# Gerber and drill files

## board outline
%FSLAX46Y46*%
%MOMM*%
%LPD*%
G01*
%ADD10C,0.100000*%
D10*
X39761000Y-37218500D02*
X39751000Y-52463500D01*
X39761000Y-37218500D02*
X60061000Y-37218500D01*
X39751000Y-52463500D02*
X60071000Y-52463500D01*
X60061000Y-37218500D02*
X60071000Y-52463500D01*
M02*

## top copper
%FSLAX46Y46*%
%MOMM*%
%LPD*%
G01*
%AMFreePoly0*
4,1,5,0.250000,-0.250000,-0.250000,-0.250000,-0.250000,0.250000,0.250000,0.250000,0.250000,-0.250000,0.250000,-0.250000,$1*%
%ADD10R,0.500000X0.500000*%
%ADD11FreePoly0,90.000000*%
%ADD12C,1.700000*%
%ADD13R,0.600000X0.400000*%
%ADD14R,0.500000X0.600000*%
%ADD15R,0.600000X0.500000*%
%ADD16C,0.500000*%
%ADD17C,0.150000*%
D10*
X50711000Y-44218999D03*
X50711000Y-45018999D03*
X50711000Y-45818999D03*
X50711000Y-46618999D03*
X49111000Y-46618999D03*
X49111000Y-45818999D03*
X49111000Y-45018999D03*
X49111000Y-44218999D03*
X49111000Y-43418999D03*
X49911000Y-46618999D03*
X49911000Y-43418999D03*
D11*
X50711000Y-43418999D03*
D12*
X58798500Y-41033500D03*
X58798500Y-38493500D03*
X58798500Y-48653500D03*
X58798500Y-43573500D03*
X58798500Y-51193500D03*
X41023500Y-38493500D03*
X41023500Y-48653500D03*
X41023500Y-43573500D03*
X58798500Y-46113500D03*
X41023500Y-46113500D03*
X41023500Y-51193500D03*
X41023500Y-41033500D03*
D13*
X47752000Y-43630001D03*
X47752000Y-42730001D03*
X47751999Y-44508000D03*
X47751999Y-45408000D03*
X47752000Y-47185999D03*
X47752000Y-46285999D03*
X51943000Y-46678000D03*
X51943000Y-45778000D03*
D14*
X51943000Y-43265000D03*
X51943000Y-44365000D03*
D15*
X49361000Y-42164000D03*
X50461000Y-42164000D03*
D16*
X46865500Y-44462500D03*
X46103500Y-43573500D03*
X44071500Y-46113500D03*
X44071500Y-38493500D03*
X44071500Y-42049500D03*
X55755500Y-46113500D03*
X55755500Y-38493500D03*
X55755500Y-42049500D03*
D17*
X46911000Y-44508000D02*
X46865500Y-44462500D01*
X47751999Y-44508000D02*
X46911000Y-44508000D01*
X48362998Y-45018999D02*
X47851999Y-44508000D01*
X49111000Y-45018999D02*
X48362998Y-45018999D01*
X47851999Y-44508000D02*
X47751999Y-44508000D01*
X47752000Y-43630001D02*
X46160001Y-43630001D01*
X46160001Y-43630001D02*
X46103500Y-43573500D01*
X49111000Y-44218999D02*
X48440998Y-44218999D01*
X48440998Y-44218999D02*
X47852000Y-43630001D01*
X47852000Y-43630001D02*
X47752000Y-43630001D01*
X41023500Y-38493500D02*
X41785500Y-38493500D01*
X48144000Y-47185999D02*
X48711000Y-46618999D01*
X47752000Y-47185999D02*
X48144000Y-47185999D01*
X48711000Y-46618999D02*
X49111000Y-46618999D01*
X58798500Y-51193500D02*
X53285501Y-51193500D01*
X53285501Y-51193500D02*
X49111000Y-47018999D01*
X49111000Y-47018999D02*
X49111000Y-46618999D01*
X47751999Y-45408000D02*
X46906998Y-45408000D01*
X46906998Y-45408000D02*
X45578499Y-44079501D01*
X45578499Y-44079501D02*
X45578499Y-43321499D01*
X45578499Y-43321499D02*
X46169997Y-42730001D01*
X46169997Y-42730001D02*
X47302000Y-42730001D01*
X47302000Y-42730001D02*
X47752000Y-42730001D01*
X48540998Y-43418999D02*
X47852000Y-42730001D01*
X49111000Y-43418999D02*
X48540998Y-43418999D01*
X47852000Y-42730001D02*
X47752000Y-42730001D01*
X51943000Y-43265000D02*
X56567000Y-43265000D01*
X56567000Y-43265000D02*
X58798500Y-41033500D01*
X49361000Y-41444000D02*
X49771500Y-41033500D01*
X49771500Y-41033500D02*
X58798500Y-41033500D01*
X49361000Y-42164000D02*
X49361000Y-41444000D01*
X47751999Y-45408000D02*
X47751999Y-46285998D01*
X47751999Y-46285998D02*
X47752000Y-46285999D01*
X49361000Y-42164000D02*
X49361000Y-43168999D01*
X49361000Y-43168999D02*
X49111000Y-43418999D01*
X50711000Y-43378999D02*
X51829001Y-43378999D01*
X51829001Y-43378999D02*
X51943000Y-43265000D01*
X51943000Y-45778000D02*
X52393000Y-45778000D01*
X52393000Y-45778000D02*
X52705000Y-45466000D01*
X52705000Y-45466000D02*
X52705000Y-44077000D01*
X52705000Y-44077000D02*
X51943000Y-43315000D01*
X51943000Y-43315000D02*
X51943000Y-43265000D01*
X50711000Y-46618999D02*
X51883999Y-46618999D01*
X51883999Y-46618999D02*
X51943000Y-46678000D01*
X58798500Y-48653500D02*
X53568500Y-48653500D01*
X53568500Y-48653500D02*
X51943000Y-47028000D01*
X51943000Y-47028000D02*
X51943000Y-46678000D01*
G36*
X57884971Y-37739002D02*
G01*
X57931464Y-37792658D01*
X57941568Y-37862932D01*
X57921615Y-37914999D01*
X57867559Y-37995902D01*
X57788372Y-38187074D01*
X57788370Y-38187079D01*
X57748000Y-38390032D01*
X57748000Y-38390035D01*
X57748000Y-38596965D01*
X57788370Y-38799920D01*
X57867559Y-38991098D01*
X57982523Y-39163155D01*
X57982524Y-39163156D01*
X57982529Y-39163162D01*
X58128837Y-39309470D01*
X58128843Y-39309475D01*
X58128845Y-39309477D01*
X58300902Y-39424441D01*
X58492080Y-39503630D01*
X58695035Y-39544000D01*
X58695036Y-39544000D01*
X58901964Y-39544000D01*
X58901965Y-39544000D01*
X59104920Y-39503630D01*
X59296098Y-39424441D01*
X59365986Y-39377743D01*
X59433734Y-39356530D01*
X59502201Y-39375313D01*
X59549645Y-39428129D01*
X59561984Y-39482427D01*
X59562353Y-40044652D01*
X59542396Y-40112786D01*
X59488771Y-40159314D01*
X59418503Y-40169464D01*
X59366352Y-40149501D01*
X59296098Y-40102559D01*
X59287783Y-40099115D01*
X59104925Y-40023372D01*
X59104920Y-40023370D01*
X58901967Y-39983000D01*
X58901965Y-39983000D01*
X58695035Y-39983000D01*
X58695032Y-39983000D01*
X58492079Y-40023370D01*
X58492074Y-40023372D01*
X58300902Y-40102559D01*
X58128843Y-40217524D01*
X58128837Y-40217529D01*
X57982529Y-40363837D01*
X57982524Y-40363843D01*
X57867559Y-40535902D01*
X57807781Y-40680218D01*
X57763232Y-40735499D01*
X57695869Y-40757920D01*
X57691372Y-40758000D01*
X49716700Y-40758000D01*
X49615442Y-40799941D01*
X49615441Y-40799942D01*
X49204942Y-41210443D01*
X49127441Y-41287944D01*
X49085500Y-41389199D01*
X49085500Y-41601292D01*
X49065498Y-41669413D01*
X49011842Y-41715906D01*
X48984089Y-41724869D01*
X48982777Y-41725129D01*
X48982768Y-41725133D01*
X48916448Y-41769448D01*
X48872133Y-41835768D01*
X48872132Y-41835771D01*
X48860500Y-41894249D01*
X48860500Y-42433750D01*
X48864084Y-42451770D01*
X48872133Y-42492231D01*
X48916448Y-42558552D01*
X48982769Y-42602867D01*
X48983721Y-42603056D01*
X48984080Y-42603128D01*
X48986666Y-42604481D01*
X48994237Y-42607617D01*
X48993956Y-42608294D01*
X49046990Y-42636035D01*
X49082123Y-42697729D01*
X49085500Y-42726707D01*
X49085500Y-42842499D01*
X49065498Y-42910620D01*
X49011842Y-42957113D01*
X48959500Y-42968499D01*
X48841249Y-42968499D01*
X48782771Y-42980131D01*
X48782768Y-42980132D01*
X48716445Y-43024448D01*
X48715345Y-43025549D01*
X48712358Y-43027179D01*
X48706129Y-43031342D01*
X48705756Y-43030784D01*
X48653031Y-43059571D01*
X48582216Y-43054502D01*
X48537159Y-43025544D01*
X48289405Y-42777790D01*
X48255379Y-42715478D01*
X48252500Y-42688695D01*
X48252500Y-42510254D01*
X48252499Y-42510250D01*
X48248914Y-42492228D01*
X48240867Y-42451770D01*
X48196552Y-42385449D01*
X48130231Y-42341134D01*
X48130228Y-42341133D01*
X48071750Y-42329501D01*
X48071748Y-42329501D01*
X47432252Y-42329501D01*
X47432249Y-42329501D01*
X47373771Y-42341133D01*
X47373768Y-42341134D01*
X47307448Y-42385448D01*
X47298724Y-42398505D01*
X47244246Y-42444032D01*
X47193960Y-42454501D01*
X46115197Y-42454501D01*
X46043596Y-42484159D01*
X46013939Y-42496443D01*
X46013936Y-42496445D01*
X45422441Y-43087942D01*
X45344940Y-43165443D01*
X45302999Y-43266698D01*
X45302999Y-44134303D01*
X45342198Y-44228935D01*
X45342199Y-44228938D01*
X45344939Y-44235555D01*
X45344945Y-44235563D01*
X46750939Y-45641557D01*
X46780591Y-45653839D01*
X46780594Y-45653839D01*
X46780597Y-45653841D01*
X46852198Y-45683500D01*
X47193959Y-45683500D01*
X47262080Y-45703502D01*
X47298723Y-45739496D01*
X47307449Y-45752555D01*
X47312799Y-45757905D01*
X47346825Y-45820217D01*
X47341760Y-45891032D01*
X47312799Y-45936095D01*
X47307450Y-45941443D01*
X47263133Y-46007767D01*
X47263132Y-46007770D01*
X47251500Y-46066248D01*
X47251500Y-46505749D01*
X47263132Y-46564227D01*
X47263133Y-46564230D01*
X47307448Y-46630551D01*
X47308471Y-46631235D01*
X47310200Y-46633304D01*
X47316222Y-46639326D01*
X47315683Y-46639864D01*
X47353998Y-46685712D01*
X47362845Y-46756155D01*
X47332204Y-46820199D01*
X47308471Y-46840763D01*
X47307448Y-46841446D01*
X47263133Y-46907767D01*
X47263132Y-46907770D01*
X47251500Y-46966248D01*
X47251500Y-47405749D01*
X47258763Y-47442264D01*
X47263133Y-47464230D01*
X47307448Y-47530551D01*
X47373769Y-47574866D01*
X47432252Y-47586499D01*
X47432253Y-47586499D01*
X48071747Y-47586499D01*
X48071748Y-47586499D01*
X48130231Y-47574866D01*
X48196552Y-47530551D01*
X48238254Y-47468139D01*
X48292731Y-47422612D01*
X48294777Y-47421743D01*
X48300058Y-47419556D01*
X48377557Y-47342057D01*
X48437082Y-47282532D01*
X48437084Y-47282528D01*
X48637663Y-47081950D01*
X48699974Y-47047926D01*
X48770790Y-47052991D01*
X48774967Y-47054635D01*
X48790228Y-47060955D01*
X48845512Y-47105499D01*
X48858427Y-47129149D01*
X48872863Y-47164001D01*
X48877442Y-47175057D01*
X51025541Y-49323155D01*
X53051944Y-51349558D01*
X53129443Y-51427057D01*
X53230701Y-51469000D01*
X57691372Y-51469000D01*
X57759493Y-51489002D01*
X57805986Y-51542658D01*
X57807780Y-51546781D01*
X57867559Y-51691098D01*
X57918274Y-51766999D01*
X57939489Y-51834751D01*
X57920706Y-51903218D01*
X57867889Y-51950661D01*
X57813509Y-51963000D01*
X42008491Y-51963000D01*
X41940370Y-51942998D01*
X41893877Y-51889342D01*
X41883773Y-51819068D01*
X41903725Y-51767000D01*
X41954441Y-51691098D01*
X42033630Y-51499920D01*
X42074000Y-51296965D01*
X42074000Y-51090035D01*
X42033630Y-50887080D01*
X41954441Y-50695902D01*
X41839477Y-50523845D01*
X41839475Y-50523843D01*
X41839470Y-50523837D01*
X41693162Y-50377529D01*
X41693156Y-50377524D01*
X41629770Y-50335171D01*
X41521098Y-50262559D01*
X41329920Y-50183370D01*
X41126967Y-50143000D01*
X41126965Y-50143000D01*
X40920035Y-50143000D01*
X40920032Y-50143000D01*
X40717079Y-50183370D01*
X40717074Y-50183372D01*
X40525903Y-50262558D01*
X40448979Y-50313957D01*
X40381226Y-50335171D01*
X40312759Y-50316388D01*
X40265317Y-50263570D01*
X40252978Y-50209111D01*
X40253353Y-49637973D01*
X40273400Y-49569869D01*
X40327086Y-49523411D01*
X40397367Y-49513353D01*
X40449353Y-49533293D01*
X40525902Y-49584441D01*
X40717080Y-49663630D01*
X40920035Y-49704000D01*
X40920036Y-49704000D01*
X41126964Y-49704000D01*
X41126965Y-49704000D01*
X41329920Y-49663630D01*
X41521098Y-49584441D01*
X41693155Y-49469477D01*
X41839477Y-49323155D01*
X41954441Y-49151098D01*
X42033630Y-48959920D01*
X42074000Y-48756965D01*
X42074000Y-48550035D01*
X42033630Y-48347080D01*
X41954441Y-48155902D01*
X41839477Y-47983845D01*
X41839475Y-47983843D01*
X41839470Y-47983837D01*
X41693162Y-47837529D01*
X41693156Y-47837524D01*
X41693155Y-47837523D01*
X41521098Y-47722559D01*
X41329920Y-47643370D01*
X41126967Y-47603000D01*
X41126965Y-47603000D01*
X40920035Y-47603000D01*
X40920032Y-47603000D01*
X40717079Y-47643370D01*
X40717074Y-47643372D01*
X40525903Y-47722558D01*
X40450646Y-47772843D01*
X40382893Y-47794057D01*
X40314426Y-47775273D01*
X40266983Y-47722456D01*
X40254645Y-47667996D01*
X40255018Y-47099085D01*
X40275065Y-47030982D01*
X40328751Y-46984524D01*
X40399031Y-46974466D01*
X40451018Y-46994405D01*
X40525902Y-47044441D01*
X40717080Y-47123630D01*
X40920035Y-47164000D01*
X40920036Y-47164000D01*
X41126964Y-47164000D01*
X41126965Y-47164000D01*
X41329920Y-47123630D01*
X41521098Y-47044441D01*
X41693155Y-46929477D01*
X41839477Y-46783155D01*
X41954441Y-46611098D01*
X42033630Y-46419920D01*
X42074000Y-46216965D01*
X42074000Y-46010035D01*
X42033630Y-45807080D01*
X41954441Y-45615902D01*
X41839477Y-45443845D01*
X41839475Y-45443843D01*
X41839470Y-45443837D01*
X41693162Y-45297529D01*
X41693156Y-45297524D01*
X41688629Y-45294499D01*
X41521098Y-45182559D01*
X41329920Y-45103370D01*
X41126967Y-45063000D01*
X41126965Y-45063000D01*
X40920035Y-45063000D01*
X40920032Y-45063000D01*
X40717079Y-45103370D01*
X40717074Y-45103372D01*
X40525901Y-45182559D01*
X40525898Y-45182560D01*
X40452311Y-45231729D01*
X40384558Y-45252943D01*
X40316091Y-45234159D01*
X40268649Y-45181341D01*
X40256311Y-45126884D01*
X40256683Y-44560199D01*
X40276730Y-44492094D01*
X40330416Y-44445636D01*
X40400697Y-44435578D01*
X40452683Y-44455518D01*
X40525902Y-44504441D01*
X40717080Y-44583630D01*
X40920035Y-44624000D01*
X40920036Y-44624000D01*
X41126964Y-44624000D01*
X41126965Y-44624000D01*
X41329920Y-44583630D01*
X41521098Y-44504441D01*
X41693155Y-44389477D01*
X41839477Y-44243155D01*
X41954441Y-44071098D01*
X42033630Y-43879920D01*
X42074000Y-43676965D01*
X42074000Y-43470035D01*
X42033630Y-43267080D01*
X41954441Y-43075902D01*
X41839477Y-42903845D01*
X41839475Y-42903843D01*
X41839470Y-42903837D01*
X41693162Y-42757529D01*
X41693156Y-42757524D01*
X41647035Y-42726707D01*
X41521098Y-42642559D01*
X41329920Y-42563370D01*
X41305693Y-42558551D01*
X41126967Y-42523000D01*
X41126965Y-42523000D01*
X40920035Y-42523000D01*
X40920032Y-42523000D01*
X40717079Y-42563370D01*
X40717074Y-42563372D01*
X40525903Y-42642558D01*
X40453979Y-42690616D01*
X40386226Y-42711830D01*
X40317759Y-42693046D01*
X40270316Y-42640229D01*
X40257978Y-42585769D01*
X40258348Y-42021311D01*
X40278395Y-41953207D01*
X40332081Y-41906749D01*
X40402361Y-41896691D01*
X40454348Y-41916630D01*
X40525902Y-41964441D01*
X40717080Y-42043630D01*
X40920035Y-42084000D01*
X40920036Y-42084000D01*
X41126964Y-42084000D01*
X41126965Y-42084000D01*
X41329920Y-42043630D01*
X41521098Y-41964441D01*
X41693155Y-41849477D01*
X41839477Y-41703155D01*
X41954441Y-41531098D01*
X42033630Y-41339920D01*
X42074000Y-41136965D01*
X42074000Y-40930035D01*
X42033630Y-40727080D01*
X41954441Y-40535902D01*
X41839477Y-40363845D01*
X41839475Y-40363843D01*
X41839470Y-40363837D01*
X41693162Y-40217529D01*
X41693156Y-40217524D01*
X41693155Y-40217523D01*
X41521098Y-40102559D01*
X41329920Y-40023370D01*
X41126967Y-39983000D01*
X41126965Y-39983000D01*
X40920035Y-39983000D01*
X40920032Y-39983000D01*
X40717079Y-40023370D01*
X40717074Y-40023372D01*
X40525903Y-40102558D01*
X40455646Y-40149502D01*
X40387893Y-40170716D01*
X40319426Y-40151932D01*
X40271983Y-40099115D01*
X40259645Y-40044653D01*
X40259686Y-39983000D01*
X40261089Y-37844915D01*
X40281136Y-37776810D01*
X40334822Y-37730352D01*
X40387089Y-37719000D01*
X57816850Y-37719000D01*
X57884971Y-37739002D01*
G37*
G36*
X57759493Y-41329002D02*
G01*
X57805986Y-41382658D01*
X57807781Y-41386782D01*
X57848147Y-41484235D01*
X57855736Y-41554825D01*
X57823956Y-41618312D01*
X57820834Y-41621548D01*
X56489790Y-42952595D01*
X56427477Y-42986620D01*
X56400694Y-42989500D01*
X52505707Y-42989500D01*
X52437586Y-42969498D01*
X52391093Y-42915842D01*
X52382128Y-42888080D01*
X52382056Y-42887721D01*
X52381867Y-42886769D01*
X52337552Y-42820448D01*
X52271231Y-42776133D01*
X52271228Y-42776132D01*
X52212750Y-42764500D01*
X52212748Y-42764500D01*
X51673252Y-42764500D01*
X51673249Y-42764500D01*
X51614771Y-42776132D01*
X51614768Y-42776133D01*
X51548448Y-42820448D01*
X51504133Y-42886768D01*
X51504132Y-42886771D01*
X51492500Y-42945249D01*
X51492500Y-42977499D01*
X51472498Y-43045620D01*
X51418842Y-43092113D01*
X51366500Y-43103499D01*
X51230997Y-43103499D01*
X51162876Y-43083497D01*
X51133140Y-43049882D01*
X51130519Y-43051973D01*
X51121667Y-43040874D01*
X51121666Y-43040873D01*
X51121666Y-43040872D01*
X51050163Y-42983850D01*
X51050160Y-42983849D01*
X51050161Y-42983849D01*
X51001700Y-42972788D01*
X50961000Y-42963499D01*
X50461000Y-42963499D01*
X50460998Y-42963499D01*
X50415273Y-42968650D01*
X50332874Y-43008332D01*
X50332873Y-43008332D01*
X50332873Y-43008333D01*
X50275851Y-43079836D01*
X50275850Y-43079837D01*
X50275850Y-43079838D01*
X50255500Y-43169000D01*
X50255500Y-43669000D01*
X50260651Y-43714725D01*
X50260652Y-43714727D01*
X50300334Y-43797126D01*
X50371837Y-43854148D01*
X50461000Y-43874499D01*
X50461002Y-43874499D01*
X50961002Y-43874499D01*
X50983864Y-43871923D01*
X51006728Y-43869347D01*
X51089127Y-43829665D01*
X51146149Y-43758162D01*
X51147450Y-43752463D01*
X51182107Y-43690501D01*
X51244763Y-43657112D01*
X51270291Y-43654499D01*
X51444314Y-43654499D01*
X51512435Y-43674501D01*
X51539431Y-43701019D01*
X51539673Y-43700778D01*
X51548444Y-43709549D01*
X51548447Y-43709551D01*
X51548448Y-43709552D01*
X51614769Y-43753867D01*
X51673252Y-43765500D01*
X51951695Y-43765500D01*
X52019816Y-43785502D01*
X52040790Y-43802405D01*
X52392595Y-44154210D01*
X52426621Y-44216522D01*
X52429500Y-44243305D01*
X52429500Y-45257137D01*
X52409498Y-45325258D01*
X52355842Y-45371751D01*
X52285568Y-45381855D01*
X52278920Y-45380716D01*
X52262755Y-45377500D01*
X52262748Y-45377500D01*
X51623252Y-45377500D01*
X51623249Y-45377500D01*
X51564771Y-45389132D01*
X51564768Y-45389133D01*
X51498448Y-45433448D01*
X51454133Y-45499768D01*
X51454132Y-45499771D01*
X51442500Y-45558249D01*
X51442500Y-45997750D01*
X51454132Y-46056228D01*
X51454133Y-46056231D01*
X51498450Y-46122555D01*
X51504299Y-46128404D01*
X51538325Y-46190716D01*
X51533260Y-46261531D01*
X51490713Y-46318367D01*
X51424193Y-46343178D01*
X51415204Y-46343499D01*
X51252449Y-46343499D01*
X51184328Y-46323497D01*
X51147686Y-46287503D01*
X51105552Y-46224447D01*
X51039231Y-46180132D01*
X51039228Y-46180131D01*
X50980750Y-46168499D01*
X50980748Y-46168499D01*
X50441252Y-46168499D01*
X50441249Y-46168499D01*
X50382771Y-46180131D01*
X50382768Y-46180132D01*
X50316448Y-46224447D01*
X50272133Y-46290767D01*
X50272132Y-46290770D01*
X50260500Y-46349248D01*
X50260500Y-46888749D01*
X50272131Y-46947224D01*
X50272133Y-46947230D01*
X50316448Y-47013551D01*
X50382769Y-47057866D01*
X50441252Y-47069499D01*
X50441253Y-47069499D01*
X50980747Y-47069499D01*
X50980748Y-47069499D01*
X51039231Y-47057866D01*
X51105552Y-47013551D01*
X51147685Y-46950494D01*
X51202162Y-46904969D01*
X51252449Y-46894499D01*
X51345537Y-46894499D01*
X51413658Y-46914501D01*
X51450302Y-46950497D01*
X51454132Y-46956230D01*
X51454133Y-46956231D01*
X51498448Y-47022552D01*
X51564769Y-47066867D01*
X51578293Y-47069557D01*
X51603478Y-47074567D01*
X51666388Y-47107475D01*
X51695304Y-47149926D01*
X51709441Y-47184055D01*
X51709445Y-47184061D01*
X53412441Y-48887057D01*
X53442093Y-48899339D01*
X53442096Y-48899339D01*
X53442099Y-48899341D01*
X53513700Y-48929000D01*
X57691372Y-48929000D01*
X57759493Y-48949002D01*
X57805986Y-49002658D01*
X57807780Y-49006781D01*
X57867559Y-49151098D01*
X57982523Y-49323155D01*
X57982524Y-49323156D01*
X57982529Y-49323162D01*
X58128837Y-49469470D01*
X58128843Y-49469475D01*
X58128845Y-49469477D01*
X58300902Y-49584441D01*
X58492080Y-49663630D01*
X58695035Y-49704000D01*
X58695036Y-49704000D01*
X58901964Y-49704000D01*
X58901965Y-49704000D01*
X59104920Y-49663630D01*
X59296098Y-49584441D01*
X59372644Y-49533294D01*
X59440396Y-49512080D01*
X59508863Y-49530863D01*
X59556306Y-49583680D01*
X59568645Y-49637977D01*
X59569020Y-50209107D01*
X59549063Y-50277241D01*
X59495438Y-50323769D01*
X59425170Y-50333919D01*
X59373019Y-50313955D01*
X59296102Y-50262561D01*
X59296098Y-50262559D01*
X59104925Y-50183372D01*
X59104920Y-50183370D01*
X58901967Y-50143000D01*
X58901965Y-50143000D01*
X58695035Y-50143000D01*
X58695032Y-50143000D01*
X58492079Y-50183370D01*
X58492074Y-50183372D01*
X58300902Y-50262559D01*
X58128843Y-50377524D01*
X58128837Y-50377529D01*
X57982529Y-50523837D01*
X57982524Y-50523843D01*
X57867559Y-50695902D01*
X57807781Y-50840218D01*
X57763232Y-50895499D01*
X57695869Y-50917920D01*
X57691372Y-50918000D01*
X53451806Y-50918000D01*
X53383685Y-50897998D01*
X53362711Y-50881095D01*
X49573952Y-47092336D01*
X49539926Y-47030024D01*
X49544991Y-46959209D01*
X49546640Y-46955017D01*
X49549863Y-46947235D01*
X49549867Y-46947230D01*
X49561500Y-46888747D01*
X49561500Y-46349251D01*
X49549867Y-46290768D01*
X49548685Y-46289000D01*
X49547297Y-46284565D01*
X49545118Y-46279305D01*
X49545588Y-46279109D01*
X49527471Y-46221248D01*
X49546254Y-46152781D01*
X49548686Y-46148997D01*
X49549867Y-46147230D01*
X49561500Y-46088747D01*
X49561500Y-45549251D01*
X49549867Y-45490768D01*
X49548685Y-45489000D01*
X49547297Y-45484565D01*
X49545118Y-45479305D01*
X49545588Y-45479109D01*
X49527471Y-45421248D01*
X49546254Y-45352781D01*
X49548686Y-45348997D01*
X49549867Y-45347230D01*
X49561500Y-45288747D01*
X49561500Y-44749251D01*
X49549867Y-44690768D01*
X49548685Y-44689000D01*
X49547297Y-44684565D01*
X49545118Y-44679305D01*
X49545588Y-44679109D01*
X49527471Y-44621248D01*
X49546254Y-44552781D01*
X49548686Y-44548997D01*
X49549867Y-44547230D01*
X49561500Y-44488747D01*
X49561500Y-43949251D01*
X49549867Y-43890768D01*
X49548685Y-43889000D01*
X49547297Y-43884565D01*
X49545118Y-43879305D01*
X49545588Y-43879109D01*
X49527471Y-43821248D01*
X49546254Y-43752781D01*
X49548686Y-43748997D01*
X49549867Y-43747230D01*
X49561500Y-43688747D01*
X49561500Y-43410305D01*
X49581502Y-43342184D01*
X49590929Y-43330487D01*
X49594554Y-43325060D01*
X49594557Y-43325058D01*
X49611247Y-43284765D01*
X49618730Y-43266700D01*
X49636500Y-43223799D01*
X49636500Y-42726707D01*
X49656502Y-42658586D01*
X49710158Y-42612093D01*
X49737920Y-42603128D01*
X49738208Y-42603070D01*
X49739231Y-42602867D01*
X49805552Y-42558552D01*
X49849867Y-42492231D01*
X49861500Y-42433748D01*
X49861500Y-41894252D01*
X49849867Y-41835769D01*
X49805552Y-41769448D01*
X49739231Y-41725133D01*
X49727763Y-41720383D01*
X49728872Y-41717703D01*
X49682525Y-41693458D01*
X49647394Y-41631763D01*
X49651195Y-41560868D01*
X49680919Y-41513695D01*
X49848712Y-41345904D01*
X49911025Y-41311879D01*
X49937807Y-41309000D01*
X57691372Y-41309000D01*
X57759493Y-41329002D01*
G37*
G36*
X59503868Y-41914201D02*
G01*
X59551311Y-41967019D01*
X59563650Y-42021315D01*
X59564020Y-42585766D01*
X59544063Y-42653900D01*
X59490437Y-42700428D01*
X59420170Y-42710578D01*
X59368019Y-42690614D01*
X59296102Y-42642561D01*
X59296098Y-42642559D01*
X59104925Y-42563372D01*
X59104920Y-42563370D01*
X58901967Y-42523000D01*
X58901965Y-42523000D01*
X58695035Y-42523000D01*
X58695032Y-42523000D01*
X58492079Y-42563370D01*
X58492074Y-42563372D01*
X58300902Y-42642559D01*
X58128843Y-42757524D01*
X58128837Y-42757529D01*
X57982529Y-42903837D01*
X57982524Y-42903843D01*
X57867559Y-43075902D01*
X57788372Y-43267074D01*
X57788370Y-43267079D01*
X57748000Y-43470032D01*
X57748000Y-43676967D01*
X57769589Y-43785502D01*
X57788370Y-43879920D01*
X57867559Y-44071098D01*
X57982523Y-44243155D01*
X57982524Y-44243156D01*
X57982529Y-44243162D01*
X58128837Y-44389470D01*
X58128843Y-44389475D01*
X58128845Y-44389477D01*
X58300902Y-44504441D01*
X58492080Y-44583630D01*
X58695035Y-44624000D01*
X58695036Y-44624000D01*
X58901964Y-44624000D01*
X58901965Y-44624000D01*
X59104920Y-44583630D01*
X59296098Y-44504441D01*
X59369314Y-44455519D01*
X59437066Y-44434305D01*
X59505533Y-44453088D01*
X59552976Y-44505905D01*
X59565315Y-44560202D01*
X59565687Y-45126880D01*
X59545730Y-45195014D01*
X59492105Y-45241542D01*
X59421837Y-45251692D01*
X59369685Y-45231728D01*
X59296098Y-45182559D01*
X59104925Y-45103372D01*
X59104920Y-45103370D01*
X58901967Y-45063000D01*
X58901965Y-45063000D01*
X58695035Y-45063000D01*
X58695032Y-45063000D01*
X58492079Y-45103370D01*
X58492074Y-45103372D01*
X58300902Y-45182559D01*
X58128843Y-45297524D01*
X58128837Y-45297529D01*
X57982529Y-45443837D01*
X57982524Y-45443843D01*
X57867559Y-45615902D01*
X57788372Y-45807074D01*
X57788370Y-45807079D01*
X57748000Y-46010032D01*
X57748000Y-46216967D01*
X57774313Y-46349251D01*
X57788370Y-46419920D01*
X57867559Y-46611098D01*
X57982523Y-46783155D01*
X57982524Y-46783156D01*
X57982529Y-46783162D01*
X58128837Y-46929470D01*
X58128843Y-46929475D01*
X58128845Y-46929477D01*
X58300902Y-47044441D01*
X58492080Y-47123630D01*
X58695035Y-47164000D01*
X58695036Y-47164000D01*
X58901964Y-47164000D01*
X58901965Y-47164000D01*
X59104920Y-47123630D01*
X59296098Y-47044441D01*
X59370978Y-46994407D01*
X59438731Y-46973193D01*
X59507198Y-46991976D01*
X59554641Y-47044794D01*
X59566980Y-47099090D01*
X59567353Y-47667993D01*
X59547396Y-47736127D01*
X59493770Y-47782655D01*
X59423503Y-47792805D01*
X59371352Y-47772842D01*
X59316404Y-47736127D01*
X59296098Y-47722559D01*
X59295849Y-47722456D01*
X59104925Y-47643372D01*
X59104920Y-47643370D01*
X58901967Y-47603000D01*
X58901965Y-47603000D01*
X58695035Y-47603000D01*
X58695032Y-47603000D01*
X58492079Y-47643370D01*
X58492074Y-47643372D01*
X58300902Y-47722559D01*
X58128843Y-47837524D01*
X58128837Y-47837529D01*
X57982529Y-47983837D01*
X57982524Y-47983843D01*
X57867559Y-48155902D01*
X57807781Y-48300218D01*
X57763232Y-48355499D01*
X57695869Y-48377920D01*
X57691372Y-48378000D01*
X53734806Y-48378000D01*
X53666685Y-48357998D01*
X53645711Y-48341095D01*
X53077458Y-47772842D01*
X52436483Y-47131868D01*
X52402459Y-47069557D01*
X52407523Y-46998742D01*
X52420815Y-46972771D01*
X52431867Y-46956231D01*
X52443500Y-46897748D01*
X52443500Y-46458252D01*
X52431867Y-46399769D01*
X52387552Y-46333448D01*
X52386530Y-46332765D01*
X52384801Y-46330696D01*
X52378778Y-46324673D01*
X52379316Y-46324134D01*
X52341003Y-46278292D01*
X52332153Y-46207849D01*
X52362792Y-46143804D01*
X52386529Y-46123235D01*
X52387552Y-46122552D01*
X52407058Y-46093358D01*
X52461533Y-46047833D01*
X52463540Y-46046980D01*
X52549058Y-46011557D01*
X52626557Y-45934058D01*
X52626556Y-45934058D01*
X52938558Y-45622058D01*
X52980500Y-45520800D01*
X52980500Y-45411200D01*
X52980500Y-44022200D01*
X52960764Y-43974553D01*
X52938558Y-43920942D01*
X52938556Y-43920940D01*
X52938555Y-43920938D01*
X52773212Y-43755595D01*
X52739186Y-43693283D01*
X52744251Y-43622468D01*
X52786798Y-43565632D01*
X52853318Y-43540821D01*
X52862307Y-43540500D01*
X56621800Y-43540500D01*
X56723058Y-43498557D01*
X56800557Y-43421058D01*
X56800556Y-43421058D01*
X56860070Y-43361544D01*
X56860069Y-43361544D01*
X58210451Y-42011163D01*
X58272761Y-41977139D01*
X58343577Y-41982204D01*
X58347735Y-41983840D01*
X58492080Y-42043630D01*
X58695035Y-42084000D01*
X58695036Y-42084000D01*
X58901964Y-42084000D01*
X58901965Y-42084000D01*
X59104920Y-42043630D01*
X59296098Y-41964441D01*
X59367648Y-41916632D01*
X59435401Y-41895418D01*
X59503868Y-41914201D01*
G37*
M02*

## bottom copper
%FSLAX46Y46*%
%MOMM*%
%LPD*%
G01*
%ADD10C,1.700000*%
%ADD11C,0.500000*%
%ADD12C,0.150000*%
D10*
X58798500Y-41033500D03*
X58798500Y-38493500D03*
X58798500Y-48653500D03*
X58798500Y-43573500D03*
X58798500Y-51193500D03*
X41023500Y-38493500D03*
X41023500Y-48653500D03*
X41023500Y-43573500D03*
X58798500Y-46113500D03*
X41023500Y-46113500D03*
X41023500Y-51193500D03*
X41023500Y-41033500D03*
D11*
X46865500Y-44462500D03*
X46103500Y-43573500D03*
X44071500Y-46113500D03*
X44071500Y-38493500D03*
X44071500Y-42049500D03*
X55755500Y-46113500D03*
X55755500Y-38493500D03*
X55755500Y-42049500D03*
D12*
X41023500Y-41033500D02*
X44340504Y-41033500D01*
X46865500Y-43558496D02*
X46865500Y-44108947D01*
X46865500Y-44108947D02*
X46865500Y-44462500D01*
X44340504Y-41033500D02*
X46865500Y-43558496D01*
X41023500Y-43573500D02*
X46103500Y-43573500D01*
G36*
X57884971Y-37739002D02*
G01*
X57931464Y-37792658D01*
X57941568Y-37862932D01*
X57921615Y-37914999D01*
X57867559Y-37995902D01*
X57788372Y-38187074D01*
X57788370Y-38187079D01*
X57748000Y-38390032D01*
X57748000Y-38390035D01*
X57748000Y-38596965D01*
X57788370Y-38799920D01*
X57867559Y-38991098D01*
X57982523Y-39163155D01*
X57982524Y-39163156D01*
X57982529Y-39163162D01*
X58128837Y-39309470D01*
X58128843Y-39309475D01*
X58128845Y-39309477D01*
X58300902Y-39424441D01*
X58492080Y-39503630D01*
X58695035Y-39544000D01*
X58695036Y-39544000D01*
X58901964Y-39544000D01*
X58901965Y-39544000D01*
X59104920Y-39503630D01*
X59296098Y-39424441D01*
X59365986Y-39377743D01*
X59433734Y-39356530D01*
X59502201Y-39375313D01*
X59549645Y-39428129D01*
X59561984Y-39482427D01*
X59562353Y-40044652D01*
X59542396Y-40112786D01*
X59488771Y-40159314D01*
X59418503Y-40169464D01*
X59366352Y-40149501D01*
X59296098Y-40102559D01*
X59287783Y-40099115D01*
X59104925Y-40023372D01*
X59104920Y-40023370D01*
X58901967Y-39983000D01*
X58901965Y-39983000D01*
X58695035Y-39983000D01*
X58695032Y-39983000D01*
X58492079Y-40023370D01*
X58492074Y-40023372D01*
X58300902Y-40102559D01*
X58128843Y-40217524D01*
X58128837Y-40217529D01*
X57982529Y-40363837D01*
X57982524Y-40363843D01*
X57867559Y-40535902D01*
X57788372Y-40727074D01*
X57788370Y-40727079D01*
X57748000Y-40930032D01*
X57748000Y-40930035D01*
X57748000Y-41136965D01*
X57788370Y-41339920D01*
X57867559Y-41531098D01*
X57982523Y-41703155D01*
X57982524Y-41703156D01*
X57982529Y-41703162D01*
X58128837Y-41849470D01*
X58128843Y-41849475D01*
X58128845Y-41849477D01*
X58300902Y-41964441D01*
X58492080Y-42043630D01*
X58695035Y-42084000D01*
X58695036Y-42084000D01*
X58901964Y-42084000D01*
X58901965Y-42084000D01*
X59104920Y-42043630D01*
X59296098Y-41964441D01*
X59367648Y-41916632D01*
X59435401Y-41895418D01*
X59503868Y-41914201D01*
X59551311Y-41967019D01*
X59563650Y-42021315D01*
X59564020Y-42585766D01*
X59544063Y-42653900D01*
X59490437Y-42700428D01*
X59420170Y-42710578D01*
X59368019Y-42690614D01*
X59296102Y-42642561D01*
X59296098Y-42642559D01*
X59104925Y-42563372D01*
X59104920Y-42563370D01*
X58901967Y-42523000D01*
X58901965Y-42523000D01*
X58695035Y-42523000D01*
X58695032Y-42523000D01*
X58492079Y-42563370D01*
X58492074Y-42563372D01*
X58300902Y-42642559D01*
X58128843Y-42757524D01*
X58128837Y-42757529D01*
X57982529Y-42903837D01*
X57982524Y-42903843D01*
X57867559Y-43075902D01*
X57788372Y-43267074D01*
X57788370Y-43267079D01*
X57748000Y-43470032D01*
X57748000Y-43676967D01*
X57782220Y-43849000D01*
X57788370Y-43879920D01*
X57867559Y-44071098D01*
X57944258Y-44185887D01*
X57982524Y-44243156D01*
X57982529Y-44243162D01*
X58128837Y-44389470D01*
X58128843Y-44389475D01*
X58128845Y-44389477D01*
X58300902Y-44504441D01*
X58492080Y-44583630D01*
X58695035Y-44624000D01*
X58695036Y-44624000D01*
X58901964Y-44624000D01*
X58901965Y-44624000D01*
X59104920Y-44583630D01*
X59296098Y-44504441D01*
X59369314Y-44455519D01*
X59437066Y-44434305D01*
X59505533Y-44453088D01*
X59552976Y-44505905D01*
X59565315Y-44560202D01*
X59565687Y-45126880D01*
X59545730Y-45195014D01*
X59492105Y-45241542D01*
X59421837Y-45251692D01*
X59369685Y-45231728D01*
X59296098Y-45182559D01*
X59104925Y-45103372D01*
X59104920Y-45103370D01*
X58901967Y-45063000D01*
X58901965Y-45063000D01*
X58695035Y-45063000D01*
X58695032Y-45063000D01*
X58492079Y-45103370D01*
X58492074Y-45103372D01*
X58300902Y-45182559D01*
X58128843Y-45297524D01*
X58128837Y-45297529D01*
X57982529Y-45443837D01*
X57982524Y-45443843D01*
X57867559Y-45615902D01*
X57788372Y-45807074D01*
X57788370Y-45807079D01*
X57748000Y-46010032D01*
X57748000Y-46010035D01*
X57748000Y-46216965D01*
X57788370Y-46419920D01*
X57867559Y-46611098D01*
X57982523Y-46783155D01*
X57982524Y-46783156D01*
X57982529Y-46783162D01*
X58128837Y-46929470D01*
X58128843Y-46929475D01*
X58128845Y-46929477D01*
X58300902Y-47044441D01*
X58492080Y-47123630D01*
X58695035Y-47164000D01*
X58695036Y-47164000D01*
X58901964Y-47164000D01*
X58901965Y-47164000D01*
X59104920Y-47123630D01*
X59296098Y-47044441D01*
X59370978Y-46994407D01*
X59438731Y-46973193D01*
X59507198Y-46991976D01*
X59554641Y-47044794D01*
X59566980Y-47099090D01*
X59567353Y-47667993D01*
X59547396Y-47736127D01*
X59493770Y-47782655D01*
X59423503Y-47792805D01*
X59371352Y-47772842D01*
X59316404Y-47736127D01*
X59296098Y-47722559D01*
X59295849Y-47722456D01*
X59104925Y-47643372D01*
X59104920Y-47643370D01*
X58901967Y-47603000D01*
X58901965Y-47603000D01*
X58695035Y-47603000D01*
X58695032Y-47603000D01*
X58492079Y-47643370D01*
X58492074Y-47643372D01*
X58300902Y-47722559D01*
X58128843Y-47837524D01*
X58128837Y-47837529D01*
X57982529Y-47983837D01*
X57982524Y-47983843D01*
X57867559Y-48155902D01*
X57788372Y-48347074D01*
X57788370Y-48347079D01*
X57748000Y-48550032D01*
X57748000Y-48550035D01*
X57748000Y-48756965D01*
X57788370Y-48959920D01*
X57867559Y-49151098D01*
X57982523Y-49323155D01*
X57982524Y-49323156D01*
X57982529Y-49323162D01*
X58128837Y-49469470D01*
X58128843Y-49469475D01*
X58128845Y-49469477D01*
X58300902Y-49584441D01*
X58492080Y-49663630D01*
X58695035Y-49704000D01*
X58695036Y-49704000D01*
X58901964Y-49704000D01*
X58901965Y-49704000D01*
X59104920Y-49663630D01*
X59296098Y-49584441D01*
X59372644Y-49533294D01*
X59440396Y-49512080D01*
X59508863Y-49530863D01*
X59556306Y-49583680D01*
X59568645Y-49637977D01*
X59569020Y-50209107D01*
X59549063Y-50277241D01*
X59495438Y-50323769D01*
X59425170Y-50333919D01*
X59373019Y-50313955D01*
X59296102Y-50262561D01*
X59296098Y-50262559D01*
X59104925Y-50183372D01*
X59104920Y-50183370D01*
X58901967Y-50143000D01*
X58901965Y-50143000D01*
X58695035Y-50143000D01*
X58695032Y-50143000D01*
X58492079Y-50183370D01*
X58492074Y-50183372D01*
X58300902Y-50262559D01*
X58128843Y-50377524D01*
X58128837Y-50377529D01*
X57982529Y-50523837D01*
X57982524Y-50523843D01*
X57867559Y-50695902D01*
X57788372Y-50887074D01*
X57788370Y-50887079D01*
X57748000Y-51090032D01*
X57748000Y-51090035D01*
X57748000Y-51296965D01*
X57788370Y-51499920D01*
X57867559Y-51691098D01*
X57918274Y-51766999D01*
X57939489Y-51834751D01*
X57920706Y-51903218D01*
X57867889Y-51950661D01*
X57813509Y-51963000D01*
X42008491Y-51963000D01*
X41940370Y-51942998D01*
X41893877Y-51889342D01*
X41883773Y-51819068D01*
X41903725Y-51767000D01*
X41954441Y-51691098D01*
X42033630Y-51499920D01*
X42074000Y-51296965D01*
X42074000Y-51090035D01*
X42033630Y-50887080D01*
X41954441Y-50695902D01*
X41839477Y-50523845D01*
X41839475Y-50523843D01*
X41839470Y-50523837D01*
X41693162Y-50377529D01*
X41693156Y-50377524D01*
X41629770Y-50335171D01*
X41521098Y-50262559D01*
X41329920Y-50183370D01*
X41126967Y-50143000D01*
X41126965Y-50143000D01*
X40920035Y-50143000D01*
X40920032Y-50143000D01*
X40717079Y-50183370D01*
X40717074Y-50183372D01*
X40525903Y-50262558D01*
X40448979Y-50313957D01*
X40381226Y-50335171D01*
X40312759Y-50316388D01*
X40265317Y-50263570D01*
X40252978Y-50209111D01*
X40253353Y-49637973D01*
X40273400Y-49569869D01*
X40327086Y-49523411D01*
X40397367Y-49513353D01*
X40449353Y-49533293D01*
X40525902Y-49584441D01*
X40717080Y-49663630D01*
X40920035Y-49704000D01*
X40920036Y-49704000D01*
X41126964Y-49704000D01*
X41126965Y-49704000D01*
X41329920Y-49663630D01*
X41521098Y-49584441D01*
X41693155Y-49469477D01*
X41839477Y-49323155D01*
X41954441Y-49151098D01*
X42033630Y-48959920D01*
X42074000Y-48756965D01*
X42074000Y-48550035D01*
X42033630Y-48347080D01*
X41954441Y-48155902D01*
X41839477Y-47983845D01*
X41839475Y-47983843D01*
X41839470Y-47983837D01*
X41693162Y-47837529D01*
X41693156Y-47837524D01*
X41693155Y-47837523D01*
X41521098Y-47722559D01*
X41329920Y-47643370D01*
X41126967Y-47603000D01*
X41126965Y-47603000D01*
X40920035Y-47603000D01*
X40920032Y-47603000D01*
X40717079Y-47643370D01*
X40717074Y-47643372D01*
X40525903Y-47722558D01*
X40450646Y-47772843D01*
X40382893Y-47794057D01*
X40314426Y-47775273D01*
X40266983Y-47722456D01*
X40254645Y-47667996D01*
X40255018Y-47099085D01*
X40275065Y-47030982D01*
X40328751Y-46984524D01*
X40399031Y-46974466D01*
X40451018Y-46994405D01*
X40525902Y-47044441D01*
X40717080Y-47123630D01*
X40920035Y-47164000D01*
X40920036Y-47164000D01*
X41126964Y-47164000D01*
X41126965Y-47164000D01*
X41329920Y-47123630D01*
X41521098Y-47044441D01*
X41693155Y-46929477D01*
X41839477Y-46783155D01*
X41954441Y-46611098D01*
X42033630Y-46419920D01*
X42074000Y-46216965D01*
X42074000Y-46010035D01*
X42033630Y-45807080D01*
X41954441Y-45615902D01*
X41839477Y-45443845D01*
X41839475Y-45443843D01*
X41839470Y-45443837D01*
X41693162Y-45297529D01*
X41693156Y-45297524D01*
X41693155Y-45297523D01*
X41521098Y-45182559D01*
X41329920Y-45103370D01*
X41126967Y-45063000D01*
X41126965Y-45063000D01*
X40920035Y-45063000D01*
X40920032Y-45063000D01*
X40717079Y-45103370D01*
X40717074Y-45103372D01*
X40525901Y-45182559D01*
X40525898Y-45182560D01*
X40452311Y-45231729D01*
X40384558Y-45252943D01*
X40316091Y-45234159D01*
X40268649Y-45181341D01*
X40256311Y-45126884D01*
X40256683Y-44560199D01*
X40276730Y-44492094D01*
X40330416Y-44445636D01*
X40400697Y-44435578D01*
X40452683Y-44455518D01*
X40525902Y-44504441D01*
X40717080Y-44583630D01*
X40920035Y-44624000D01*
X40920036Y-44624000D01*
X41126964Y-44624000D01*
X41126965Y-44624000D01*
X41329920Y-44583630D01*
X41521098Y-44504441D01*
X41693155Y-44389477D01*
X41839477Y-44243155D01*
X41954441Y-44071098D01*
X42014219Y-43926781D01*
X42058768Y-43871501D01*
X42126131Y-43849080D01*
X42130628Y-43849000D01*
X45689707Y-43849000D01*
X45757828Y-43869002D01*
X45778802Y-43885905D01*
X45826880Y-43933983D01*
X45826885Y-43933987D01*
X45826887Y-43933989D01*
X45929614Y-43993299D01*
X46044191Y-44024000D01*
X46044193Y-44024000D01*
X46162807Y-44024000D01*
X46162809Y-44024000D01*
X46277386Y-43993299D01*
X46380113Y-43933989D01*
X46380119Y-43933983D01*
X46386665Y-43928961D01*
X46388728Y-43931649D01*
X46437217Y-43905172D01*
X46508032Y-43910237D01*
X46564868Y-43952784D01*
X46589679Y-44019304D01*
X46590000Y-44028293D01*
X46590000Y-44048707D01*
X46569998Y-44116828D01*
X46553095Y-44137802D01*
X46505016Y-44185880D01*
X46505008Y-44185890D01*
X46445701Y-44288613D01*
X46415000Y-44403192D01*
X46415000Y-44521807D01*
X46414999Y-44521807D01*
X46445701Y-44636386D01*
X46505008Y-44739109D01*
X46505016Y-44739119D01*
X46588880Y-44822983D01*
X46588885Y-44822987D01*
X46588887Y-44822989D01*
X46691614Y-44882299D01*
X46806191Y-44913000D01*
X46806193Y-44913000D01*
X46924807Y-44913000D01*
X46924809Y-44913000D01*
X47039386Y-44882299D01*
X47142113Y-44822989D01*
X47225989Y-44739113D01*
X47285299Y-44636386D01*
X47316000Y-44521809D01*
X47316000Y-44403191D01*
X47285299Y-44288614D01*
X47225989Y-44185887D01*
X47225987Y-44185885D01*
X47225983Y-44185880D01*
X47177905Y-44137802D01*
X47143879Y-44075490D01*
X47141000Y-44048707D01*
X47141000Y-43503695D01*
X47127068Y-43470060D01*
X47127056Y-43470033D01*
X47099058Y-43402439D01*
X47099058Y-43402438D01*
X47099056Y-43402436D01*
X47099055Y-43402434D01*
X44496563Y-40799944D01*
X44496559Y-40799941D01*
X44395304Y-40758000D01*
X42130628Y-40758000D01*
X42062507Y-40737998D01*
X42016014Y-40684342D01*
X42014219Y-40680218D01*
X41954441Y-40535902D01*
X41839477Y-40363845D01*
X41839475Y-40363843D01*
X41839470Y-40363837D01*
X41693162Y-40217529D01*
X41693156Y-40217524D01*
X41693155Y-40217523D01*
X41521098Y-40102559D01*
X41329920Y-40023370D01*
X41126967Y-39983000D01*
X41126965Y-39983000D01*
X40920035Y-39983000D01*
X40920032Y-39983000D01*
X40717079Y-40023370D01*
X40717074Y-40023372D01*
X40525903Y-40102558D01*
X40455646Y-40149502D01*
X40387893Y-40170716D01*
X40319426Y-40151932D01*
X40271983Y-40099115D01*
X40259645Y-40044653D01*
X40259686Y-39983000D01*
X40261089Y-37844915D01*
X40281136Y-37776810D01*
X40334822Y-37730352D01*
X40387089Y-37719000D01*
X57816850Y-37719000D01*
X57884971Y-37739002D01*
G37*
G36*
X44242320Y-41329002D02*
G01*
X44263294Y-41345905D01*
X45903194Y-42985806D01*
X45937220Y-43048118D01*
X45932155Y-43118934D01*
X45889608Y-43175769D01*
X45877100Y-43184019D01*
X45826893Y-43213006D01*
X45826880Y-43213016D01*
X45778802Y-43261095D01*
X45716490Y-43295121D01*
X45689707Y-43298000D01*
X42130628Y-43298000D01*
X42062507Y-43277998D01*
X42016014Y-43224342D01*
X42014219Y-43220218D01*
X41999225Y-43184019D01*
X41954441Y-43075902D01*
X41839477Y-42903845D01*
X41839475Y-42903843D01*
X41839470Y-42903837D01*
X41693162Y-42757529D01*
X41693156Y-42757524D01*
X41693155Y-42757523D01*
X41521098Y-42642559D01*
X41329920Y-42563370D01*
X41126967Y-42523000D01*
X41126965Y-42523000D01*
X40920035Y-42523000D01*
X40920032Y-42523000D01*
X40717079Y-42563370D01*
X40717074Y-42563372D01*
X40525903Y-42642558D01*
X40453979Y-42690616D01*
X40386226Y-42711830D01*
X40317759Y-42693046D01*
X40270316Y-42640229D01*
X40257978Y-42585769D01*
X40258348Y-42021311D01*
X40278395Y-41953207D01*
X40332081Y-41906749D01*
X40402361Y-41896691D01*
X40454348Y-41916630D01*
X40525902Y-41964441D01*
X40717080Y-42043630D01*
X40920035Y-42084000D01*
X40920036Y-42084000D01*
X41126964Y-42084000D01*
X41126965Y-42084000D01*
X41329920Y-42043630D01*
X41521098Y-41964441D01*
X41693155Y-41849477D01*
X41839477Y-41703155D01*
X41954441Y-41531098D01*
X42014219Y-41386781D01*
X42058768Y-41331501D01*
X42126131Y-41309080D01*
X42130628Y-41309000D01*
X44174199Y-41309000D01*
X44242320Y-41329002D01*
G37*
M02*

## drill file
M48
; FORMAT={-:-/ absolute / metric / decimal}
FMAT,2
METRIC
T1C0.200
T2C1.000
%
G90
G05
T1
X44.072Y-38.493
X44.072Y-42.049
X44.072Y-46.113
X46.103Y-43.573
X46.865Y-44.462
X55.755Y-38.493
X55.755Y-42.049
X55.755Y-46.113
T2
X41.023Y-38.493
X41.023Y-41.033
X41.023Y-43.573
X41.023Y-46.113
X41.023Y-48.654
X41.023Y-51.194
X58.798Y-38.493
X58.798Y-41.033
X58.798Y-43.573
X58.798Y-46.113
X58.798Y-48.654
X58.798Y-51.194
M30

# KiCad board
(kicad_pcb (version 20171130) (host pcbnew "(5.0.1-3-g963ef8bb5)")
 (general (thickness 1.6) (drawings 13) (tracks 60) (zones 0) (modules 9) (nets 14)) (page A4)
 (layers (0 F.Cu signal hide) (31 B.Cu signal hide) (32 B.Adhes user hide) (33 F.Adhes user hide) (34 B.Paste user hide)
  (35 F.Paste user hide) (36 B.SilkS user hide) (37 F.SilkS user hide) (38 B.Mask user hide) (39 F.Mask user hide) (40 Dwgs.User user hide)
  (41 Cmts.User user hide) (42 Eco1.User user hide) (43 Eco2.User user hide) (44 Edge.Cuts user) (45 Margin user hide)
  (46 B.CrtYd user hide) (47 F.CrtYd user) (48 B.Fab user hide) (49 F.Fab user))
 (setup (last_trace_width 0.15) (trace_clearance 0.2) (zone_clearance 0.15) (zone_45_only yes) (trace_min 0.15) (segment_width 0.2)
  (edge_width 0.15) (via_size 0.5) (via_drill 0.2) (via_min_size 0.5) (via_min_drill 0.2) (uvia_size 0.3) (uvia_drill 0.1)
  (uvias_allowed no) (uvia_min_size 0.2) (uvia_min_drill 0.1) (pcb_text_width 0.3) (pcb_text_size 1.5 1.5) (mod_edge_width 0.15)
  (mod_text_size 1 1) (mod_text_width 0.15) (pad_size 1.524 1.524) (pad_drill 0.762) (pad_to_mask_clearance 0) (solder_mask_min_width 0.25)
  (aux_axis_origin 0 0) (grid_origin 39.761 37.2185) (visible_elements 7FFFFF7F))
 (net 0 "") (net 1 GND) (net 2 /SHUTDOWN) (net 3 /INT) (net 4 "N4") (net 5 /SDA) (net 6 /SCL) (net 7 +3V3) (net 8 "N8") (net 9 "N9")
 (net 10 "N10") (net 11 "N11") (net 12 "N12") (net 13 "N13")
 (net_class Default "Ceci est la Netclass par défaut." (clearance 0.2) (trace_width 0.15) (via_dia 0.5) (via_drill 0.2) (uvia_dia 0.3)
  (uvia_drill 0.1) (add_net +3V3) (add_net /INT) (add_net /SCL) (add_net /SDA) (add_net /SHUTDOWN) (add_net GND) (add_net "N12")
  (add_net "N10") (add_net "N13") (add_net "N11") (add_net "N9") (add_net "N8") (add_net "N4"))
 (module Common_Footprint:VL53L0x (layer F.Cu) (at 49.911 45.018999 90)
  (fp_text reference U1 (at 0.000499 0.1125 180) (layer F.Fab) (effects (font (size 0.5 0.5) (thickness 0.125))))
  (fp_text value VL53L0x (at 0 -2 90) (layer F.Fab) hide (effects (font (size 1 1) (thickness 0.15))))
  (pad 2 smd rect (at 0.8 0.8 90) (size 0.5 0.5) (layers F.Cu F.Paste F.Mask) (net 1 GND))
  (pad 3 smd rect (at 0 0.8 90) (size 0.5 0.5) (layers F.Cu F.Paste F.Mask) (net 1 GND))
  (pad 4 smd rect (at -0.8 0.8 90) (size 0.5 0.5) (layers F.Cu F.Paste F.Mask) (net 1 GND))
  (pad 5 smd rect (at -1.6 0.8 90) (size 0.5 0.5) (layers F.Cu F.Paste F.Mask) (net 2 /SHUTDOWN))
  (pad 7 smd rect (at -1.6 -0.8 270) (size 0.5 0.5) (layers F.Cu F.Paste F.Mask) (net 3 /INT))
  (pad 8 smd rect (at -0.8 -0.8 270) (size 0.5 0.5) (layers F.Cu F.Paste F.Mask) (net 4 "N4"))
  (pad 9 smd rect (at 0 -0.8 270) (size 0.5 0.5) (layers F.Cu F.Paste F.Mask) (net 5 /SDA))
  (pad 10 smd rect (at 0.8 -0.8 270) (size 0.5 0.5) (layers F.Cu F.Paste F.Mask) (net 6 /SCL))
  (pad 11 smd rect (at 1.6 -0.8 270) (size 0.5 0.5) (layers F.Cu F.Paste F.Mask) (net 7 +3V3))
  (pad 6 smd rect (at -1.6 0 270) (size 0.5 0.5) (layers F.Cu F.Paste F.Mask) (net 1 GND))
  (pad 12 smd rect (at 1.6 0 90) (size 0.5 0.5) (layers F.Cu F.Paste F.Mask) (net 1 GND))
  (pad 1 smd custom (at 1.6 0.8 90) (size 0.5 0.5) (layers F.Cu F.Paste F.Mask) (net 7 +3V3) (zone_connect 0)
   (options (clearance outline) (anchor rect)) (primitives)))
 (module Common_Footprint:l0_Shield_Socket (layer F.Cu) (at 49.911 44.8435)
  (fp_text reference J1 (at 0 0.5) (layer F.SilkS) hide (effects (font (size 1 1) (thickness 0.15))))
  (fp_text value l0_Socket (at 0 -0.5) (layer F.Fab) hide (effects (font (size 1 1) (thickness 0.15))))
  (fp_line (start -10.15 -7.625) (end -10.16 7.62) (layer Edge.Cuts) (width 0.1))
  (fp_line (start -10.15 -7.625) (end 10.15 -7.625) (layer Edge.Cuts) (width 0.1))
  (fp_line (start -10.16 7.62) (end 10.16 7.62) (layer Edge.Cuts) (width 0.1))
  (fp_line (start 10.15 -7.625) (end 10.16 7.62) (layer Edge.Cuts) (width 0.1))
  (pad 5 thru_hole circle (at 8.8875 -3.81 270) (size 1.7 1.7) (drill 1) (layers *.Cu *.Mask) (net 7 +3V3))
  (pad 6 thru_hole circle (at 8.8875 -6.35 270) (size 1.7 1.7) (drill 1) (layers *.Cu *.Mask) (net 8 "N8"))
  (pad 2 thru_hole circle (at 8.8875 3.81 270) (size 1.7 1.7) (drill 1) (layers *.Cu *.Mask) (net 2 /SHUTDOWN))
  (pad 4 thru_hole circle (at 8.8875 -1.27 270) (size 1.7 1.7) (drill 1) (layers *.Cu *.Mask) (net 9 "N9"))
  (pad 1 thru_hole circle (at 8.8875 6.35 270) (size 1.7 1.7) (drill 1) (layers *.Cu *.Mask) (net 3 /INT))
  (pad 7 thru_hole circle (at -8.8875 -6.35 270) (size 1.7 1.7) (drill 1) (layers *.Cu *.Mask) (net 1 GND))
  (pad 11 thru_hole circle (at -8.8875 3.81 270) (size 1.7 1.7) (drill 1) (layers *.Cu *.Mask) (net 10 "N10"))
  (pad 9 thru_hole circle (at -8.8875 -1.27 270) (size 1.7 1.7) (drill 1) (layers *.Cu *.Mask) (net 6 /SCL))
  (pad 3 thru_hole circle (at 8.8875 1.27 270) (size 1.7 1.7) (drill 1) (layers *.Cu *.Mask) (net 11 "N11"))
  (pad 10 thru_hole circle (at -8.8875 1.27 270) (size 1.7 1.7) (drill 1) (layers *.Cu *.Mask) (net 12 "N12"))
  (pad 12 thru_hole circle (at -8.8875 6.35 270) (size 1.7 1.7) (drill 1) (layers *.Cu *.Mask) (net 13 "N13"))
  (pad 8 thru_hole circle (at -8.8875 -3.81 270) (size 1.7 1.7) (drill 1) (layers *.Cu *.Mask) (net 5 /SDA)))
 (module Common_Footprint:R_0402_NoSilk (layer F.Cu) (at 47.752 43.180001 270)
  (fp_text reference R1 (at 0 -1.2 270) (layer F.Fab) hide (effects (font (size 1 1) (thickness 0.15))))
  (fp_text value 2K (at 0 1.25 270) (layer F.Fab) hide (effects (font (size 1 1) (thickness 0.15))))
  (pad 2 smd rect (at 0.45 0 270) (size 0.4 0.6) (layers F.Cu F.Paste F.Mask) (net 6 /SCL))
  (pad 1 smd rect (at -0.45 0 270) (size 0.4 0.6) (layers F.Cu F.Paste F.Mask) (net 7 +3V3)))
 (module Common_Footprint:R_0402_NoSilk (layer F.Cu) (at 47.751999 44.958 90)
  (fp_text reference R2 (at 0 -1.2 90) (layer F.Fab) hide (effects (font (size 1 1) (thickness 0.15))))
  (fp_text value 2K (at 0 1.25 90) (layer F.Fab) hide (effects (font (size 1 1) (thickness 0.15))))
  (pad 2 smd rect (at 0.45 0 90) (size 0.4 0.6) (layers F.Cu F.Paste F.Mask) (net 5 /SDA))
  (pad 1 smd rect (at -0.45 0 90) (size 0.4 0.6) (layers F.Cu F.Paste F.Mask) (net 7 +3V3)))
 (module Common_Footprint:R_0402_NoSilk (layer F.Cu) (at 47.752 46.735999 270)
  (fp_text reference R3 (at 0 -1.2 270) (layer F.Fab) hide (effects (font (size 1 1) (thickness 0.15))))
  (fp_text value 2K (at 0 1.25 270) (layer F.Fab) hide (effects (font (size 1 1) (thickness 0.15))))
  (pad 2 smd rect (at 0.45 0 270) (size 0.4 0.6) (layers F.Cu F.Paste F.Mask) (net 3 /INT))
  (pad 1 smd rect (at -0.45 0 270) (size 0.4 0.6) (layers F.Cu F.Paste F.Mask) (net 7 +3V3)))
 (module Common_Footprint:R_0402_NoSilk (layer F.Cu) (at 51.943 46.228 270)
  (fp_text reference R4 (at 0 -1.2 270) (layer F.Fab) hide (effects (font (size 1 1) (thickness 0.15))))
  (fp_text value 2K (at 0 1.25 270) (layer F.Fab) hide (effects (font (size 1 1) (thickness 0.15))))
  (pad 2 smd rect (at 0.45 0 270) (size 0.4 0.6) (layers F.Cu F.Paste F.Mask) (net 2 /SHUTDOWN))
  (pad 1 smd rect (at -0.45 0 270) (size 0.4 0.6) (layers F.Cu F.Paste F.Mask) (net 7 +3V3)))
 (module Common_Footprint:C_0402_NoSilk (layer F.Cu) (at 51.943 43.815 270)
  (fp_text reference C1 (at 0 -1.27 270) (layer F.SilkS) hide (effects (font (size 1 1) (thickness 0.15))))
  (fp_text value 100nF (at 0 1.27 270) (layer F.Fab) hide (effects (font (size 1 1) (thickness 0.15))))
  (pad 1 smd rect (at -0.55 0 270) (size 0.6 0.5) (layers F.Cu F.Paste F.Mask) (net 7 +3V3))
  (pad 2 smd rect (at 0.55 0 270) (size 0.6 0.5) (layers F.Cu F.Paste F.Mask) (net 1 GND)))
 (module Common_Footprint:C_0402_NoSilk (layer F.Cu) (at 49.911 42.164)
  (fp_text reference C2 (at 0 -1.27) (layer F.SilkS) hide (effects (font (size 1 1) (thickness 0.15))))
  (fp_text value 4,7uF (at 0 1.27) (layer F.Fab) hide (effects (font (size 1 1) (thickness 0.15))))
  (pad 1 smd rect (at -0.55 0) (size 0.6 0.5) (layers F.Cu F.Paste F.Mask) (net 7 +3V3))
  (pad 2 smd rect (at 0.55 0) (size 0.6 0.5) (layers F.Cu F.Paste F.Mask) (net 1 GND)))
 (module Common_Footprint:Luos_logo (layer F.Cu) (at 50.3485 49.1185)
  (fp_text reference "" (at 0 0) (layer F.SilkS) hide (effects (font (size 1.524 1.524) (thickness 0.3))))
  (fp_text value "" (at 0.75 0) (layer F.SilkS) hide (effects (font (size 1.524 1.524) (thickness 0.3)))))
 (segment (start 46.911 44.508) (end 46.8655 44.4625) (width 0.15) (layer F.Cu) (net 5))
 (segment (start 47.751999 44.508) (end 46.911 44.508) (width 0.15) (layer F.Cu) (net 5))
 (segment (start 41.0235 41.0335) (end 44.340504 41.0335) (width 0.15) (layer B.Cu) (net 5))
 (segment (start 46.8655 43.558496) (end 46.8655 44.108947) (width 0.15) (layer B.Cu) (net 5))
 (segment (start 46.8655 44.108947) (end 46.8655 44.4625) (width 0.15) (layer B.Cu) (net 5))
 (segment (start 44.340504 41.0335) (end 46.8655 43.558496) (width 0.15) (layer B.Cu) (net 5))
 (via (at 46.8655 44.4625) (size 0.5) (drill 0.2) (layers F.Cu B.Cu) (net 5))
 (segment (start 48.362998 45.018999) (end 47.851999 44.508) (width 0.15) (layer F.Cu) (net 5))
 (segment (start 49.111 45.018999) (end 48.362998 45.018999) (width 0.15) (layer F.Cu) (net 5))
 (segment (start 47.851999 44.508) (end 47.751999 44.508) (width 0.15) (layer F.Cu) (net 5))
 (via (at 46.1035 43.5735) (size 0.5) (drill 0.2) (layers F.Cu B.Cu) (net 6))
 (segment (start 47.752 43.630001) (end 46.160001 43.630001) (width 0.15) (layer F.Cu) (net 6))
 (segment (start 41.0235 43.5735) (end 46.1035 43.5735) (width 0.15) (layer B.Cu) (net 6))
 (segment (start 46.160001 43.630001) (end 46.1035 43.5735) (width 0.15) (layer F.Cu) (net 6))
 (segment (start 49.111 44.218999) (end 48.440998 44.218999) (width 0.15) (layer F.Cu) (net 6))
 (segment (start 48.440998 44.218999) (end 47.852 43.630001) (width 0.15) (layer F.Cu) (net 6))
 (segment (start 47.852 43.630001) (end 47.752 43.630001) (width 0.15) (layer F.Cu) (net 6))
 (segment (start 41.0235 38.4935) (end 41.7855 38.4935) (width 0.15) (layer F.Cu) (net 1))
 (via (at 44.0715 46.1135) (size 0.5) (drill 0.2) (layers F.Cu B.Cu) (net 1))
 (via (at 44.0715 38.4935) (size 0.5) (drill 0.2) (layers F.Cu B.Cu) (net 1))
 (via (at 44.0715 42.0495) (size 0.5) (drill 0.2) (layers F.Cu B.Cu) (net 1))
 (via (at 55.7555 46.1135) (size 0.5) (drill 0.2) (layers F.Cu B.Cu) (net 1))
 (via (at 55.7555 38.4935) (size 0.5) (drill 0.2) (layers F.Cu B.Cu) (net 1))
 (via (at 55.7555 42.0495) (size 0.5) (drill 0.2) (layers F.Cu B.Cu) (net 1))
 (segment (start 48.144 47.185999) (end 48.711 46.618999) (width 0.15) (layer F.Cu) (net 3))
 (segment (start 47.752 47.185999) (end 48.144 47.185999) (width 0.15) (layer F.Cu) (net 3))
 (segment (start 48.711 46.618999) (end 49.111 46.618999) (width 0.15) (layer F.Cu) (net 3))
 (segment (start 58.7985 51.1935) (end 53.285501 51.1935) (width 0.15) (layer F.Cu) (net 3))
 (segment (start 53.285501 51.1935) (end 49.111 47.018999) (width 0.15) (layer F.Cu) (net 3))
 (segment (start 49.111 47.018999) (end 49.111 46.618999) (width 0.15) (layer F.Cu) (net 3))
 (segment (start 47.751999 45.408) (end 46.906998 45.408) (width 0.15) (layer F.Cu) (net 7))
 (segment (start 46.906998 45.408) (end 45.578499 44.079501) (width 0.15) (layer F.Cu) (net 7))
 (segment (start 45.578499 44.079501) (end 45.578499 43.321499) (width 0.15) (layer F.Cu) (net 7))
 (segment (start 45.578499 43.321499) (end 46.169997 42.730001) (width 0.15) (layer F.Cu) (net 7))
 (segment (start 46.169997 42.730001) (end 47.302 42.730001) (width 0.15) (layer F.Cu) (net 7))
 (segment (start 47.302 42.730001) (end 47.752 42.730001) (width 0.15) (layer F.Cu) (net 7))
 (segment (start 48.540998 43.418999) (end 47.852 42.730001) (width 0.15) (layer F.Cu) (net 7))
 (segment (start 49.111 43.418999) (end 48.540998 43.418999) (width 0.15) (layer F.Cu) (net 7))
 (segment (start 47.852 42.730001) (end 47.752 42.730001) (width 0.15) (layer F.Cu) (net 7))
 (segment (start 51.943 43.265) (end 56.567 43.265) (width 0.15) (layer F.Cu) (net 7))
 (segment (start 56.567 43.265) (end 58.7985 41.0335) (width 0.15) (layer F.Cu) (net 7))
 (segment (start 49.361 41.444) (end 49.7715 41.0335) (width 0.15) (layer F.Cu) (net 7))
 (segment (start 49.7715 41.0335) (end 58.7985 41.0335) (width 0.15) (layer F.Cu) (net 7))
 (segment (start 49.361 42.164) (end 49.361 41.444) (width 0.15) (layer F.Cu) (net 7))
 (segment (start 47.751999 45.408) (end 47.751999 46.285998) (width 0.15) (layer F.Cu) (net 7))
 (segment (start 47.751999 46.285998) (end 47.752 46.285999) (width 0.15) (layer F.Cu) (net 7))
 (segment (start 49.361 42.164) (end 49.361 43.168999) (width 0.15) (layer F.Cu) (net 7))
 (segment (start 49.361 43.168999) (end 49.111 43.418999) (width 0.15) (layer F.Cu) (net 7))
 (segment (start 50.711 43.378999) (end 51.829001 43.378999) (width 0.15) (layer F.Cu) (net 7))
 (segment (start 51.829001 43.378999) (end 51.943 43.265) (width 0.15) (layer F.Cu) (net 7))
 (segment (start 51.943 45.778) (end 52.393 45.778) (width 0.15) (layer F.Cu) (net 7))
 (segment (start 52.393 45.778) (end 52.705 45.466) (width 0.15) (layer F.Cu) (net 7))
 (segment (start 52.705 45.466) (end 52.705 44.077) (width 0.15) (layer F.Cu) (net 7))
 (segment (start 52.705 44.077) (end 51.943 43.315) (width 0.15) (layer F.Cu) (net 7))
 (segment (start 51.943 43.315) (end 51.943 43.265) (width 0.15) (layer F.Cu) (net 7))
 (segment (start 50.711 46.618999) (end 51.883999 46.618999) (width 0.15) (layer F.Cu) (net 2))
 (segment (start 51.883999 46.618999) (end 51.943 46.678) (width 0.15) (layer F.Cu) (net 2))
 (segment (start 58.7985 48.6535) (end 53.5685 48.6535) (width 0.15) (layer F.Cu) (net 2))
 (segment (start 53.5685 48.6535) (end 51.943 47.028) (width 0.15) (layer F.Cu) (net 2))
 (segment (start 51.943 47.028) (end 51.943 46.678) (width 0.15) (layer F.Cu) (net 2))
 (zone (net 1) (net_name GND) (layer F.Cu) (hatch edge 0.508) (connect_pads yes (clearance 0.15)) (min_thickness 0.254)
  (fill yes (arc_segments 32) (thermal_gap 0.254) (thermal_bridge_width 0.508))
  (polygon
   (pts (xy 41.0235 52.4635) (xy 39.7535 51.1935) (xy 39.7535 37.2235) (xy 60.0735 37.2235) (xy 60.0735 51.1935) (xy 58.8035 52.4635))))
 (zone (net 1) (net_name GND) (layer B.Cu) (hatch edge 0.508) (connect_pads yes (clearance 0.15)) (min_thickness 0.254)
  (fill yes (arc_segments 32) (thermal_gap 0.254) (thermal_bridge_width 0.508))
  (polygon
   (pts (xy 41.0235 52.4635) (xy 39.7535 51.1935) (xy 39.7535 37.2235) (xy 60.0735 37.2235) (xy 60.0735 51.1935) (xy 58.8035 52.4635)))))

